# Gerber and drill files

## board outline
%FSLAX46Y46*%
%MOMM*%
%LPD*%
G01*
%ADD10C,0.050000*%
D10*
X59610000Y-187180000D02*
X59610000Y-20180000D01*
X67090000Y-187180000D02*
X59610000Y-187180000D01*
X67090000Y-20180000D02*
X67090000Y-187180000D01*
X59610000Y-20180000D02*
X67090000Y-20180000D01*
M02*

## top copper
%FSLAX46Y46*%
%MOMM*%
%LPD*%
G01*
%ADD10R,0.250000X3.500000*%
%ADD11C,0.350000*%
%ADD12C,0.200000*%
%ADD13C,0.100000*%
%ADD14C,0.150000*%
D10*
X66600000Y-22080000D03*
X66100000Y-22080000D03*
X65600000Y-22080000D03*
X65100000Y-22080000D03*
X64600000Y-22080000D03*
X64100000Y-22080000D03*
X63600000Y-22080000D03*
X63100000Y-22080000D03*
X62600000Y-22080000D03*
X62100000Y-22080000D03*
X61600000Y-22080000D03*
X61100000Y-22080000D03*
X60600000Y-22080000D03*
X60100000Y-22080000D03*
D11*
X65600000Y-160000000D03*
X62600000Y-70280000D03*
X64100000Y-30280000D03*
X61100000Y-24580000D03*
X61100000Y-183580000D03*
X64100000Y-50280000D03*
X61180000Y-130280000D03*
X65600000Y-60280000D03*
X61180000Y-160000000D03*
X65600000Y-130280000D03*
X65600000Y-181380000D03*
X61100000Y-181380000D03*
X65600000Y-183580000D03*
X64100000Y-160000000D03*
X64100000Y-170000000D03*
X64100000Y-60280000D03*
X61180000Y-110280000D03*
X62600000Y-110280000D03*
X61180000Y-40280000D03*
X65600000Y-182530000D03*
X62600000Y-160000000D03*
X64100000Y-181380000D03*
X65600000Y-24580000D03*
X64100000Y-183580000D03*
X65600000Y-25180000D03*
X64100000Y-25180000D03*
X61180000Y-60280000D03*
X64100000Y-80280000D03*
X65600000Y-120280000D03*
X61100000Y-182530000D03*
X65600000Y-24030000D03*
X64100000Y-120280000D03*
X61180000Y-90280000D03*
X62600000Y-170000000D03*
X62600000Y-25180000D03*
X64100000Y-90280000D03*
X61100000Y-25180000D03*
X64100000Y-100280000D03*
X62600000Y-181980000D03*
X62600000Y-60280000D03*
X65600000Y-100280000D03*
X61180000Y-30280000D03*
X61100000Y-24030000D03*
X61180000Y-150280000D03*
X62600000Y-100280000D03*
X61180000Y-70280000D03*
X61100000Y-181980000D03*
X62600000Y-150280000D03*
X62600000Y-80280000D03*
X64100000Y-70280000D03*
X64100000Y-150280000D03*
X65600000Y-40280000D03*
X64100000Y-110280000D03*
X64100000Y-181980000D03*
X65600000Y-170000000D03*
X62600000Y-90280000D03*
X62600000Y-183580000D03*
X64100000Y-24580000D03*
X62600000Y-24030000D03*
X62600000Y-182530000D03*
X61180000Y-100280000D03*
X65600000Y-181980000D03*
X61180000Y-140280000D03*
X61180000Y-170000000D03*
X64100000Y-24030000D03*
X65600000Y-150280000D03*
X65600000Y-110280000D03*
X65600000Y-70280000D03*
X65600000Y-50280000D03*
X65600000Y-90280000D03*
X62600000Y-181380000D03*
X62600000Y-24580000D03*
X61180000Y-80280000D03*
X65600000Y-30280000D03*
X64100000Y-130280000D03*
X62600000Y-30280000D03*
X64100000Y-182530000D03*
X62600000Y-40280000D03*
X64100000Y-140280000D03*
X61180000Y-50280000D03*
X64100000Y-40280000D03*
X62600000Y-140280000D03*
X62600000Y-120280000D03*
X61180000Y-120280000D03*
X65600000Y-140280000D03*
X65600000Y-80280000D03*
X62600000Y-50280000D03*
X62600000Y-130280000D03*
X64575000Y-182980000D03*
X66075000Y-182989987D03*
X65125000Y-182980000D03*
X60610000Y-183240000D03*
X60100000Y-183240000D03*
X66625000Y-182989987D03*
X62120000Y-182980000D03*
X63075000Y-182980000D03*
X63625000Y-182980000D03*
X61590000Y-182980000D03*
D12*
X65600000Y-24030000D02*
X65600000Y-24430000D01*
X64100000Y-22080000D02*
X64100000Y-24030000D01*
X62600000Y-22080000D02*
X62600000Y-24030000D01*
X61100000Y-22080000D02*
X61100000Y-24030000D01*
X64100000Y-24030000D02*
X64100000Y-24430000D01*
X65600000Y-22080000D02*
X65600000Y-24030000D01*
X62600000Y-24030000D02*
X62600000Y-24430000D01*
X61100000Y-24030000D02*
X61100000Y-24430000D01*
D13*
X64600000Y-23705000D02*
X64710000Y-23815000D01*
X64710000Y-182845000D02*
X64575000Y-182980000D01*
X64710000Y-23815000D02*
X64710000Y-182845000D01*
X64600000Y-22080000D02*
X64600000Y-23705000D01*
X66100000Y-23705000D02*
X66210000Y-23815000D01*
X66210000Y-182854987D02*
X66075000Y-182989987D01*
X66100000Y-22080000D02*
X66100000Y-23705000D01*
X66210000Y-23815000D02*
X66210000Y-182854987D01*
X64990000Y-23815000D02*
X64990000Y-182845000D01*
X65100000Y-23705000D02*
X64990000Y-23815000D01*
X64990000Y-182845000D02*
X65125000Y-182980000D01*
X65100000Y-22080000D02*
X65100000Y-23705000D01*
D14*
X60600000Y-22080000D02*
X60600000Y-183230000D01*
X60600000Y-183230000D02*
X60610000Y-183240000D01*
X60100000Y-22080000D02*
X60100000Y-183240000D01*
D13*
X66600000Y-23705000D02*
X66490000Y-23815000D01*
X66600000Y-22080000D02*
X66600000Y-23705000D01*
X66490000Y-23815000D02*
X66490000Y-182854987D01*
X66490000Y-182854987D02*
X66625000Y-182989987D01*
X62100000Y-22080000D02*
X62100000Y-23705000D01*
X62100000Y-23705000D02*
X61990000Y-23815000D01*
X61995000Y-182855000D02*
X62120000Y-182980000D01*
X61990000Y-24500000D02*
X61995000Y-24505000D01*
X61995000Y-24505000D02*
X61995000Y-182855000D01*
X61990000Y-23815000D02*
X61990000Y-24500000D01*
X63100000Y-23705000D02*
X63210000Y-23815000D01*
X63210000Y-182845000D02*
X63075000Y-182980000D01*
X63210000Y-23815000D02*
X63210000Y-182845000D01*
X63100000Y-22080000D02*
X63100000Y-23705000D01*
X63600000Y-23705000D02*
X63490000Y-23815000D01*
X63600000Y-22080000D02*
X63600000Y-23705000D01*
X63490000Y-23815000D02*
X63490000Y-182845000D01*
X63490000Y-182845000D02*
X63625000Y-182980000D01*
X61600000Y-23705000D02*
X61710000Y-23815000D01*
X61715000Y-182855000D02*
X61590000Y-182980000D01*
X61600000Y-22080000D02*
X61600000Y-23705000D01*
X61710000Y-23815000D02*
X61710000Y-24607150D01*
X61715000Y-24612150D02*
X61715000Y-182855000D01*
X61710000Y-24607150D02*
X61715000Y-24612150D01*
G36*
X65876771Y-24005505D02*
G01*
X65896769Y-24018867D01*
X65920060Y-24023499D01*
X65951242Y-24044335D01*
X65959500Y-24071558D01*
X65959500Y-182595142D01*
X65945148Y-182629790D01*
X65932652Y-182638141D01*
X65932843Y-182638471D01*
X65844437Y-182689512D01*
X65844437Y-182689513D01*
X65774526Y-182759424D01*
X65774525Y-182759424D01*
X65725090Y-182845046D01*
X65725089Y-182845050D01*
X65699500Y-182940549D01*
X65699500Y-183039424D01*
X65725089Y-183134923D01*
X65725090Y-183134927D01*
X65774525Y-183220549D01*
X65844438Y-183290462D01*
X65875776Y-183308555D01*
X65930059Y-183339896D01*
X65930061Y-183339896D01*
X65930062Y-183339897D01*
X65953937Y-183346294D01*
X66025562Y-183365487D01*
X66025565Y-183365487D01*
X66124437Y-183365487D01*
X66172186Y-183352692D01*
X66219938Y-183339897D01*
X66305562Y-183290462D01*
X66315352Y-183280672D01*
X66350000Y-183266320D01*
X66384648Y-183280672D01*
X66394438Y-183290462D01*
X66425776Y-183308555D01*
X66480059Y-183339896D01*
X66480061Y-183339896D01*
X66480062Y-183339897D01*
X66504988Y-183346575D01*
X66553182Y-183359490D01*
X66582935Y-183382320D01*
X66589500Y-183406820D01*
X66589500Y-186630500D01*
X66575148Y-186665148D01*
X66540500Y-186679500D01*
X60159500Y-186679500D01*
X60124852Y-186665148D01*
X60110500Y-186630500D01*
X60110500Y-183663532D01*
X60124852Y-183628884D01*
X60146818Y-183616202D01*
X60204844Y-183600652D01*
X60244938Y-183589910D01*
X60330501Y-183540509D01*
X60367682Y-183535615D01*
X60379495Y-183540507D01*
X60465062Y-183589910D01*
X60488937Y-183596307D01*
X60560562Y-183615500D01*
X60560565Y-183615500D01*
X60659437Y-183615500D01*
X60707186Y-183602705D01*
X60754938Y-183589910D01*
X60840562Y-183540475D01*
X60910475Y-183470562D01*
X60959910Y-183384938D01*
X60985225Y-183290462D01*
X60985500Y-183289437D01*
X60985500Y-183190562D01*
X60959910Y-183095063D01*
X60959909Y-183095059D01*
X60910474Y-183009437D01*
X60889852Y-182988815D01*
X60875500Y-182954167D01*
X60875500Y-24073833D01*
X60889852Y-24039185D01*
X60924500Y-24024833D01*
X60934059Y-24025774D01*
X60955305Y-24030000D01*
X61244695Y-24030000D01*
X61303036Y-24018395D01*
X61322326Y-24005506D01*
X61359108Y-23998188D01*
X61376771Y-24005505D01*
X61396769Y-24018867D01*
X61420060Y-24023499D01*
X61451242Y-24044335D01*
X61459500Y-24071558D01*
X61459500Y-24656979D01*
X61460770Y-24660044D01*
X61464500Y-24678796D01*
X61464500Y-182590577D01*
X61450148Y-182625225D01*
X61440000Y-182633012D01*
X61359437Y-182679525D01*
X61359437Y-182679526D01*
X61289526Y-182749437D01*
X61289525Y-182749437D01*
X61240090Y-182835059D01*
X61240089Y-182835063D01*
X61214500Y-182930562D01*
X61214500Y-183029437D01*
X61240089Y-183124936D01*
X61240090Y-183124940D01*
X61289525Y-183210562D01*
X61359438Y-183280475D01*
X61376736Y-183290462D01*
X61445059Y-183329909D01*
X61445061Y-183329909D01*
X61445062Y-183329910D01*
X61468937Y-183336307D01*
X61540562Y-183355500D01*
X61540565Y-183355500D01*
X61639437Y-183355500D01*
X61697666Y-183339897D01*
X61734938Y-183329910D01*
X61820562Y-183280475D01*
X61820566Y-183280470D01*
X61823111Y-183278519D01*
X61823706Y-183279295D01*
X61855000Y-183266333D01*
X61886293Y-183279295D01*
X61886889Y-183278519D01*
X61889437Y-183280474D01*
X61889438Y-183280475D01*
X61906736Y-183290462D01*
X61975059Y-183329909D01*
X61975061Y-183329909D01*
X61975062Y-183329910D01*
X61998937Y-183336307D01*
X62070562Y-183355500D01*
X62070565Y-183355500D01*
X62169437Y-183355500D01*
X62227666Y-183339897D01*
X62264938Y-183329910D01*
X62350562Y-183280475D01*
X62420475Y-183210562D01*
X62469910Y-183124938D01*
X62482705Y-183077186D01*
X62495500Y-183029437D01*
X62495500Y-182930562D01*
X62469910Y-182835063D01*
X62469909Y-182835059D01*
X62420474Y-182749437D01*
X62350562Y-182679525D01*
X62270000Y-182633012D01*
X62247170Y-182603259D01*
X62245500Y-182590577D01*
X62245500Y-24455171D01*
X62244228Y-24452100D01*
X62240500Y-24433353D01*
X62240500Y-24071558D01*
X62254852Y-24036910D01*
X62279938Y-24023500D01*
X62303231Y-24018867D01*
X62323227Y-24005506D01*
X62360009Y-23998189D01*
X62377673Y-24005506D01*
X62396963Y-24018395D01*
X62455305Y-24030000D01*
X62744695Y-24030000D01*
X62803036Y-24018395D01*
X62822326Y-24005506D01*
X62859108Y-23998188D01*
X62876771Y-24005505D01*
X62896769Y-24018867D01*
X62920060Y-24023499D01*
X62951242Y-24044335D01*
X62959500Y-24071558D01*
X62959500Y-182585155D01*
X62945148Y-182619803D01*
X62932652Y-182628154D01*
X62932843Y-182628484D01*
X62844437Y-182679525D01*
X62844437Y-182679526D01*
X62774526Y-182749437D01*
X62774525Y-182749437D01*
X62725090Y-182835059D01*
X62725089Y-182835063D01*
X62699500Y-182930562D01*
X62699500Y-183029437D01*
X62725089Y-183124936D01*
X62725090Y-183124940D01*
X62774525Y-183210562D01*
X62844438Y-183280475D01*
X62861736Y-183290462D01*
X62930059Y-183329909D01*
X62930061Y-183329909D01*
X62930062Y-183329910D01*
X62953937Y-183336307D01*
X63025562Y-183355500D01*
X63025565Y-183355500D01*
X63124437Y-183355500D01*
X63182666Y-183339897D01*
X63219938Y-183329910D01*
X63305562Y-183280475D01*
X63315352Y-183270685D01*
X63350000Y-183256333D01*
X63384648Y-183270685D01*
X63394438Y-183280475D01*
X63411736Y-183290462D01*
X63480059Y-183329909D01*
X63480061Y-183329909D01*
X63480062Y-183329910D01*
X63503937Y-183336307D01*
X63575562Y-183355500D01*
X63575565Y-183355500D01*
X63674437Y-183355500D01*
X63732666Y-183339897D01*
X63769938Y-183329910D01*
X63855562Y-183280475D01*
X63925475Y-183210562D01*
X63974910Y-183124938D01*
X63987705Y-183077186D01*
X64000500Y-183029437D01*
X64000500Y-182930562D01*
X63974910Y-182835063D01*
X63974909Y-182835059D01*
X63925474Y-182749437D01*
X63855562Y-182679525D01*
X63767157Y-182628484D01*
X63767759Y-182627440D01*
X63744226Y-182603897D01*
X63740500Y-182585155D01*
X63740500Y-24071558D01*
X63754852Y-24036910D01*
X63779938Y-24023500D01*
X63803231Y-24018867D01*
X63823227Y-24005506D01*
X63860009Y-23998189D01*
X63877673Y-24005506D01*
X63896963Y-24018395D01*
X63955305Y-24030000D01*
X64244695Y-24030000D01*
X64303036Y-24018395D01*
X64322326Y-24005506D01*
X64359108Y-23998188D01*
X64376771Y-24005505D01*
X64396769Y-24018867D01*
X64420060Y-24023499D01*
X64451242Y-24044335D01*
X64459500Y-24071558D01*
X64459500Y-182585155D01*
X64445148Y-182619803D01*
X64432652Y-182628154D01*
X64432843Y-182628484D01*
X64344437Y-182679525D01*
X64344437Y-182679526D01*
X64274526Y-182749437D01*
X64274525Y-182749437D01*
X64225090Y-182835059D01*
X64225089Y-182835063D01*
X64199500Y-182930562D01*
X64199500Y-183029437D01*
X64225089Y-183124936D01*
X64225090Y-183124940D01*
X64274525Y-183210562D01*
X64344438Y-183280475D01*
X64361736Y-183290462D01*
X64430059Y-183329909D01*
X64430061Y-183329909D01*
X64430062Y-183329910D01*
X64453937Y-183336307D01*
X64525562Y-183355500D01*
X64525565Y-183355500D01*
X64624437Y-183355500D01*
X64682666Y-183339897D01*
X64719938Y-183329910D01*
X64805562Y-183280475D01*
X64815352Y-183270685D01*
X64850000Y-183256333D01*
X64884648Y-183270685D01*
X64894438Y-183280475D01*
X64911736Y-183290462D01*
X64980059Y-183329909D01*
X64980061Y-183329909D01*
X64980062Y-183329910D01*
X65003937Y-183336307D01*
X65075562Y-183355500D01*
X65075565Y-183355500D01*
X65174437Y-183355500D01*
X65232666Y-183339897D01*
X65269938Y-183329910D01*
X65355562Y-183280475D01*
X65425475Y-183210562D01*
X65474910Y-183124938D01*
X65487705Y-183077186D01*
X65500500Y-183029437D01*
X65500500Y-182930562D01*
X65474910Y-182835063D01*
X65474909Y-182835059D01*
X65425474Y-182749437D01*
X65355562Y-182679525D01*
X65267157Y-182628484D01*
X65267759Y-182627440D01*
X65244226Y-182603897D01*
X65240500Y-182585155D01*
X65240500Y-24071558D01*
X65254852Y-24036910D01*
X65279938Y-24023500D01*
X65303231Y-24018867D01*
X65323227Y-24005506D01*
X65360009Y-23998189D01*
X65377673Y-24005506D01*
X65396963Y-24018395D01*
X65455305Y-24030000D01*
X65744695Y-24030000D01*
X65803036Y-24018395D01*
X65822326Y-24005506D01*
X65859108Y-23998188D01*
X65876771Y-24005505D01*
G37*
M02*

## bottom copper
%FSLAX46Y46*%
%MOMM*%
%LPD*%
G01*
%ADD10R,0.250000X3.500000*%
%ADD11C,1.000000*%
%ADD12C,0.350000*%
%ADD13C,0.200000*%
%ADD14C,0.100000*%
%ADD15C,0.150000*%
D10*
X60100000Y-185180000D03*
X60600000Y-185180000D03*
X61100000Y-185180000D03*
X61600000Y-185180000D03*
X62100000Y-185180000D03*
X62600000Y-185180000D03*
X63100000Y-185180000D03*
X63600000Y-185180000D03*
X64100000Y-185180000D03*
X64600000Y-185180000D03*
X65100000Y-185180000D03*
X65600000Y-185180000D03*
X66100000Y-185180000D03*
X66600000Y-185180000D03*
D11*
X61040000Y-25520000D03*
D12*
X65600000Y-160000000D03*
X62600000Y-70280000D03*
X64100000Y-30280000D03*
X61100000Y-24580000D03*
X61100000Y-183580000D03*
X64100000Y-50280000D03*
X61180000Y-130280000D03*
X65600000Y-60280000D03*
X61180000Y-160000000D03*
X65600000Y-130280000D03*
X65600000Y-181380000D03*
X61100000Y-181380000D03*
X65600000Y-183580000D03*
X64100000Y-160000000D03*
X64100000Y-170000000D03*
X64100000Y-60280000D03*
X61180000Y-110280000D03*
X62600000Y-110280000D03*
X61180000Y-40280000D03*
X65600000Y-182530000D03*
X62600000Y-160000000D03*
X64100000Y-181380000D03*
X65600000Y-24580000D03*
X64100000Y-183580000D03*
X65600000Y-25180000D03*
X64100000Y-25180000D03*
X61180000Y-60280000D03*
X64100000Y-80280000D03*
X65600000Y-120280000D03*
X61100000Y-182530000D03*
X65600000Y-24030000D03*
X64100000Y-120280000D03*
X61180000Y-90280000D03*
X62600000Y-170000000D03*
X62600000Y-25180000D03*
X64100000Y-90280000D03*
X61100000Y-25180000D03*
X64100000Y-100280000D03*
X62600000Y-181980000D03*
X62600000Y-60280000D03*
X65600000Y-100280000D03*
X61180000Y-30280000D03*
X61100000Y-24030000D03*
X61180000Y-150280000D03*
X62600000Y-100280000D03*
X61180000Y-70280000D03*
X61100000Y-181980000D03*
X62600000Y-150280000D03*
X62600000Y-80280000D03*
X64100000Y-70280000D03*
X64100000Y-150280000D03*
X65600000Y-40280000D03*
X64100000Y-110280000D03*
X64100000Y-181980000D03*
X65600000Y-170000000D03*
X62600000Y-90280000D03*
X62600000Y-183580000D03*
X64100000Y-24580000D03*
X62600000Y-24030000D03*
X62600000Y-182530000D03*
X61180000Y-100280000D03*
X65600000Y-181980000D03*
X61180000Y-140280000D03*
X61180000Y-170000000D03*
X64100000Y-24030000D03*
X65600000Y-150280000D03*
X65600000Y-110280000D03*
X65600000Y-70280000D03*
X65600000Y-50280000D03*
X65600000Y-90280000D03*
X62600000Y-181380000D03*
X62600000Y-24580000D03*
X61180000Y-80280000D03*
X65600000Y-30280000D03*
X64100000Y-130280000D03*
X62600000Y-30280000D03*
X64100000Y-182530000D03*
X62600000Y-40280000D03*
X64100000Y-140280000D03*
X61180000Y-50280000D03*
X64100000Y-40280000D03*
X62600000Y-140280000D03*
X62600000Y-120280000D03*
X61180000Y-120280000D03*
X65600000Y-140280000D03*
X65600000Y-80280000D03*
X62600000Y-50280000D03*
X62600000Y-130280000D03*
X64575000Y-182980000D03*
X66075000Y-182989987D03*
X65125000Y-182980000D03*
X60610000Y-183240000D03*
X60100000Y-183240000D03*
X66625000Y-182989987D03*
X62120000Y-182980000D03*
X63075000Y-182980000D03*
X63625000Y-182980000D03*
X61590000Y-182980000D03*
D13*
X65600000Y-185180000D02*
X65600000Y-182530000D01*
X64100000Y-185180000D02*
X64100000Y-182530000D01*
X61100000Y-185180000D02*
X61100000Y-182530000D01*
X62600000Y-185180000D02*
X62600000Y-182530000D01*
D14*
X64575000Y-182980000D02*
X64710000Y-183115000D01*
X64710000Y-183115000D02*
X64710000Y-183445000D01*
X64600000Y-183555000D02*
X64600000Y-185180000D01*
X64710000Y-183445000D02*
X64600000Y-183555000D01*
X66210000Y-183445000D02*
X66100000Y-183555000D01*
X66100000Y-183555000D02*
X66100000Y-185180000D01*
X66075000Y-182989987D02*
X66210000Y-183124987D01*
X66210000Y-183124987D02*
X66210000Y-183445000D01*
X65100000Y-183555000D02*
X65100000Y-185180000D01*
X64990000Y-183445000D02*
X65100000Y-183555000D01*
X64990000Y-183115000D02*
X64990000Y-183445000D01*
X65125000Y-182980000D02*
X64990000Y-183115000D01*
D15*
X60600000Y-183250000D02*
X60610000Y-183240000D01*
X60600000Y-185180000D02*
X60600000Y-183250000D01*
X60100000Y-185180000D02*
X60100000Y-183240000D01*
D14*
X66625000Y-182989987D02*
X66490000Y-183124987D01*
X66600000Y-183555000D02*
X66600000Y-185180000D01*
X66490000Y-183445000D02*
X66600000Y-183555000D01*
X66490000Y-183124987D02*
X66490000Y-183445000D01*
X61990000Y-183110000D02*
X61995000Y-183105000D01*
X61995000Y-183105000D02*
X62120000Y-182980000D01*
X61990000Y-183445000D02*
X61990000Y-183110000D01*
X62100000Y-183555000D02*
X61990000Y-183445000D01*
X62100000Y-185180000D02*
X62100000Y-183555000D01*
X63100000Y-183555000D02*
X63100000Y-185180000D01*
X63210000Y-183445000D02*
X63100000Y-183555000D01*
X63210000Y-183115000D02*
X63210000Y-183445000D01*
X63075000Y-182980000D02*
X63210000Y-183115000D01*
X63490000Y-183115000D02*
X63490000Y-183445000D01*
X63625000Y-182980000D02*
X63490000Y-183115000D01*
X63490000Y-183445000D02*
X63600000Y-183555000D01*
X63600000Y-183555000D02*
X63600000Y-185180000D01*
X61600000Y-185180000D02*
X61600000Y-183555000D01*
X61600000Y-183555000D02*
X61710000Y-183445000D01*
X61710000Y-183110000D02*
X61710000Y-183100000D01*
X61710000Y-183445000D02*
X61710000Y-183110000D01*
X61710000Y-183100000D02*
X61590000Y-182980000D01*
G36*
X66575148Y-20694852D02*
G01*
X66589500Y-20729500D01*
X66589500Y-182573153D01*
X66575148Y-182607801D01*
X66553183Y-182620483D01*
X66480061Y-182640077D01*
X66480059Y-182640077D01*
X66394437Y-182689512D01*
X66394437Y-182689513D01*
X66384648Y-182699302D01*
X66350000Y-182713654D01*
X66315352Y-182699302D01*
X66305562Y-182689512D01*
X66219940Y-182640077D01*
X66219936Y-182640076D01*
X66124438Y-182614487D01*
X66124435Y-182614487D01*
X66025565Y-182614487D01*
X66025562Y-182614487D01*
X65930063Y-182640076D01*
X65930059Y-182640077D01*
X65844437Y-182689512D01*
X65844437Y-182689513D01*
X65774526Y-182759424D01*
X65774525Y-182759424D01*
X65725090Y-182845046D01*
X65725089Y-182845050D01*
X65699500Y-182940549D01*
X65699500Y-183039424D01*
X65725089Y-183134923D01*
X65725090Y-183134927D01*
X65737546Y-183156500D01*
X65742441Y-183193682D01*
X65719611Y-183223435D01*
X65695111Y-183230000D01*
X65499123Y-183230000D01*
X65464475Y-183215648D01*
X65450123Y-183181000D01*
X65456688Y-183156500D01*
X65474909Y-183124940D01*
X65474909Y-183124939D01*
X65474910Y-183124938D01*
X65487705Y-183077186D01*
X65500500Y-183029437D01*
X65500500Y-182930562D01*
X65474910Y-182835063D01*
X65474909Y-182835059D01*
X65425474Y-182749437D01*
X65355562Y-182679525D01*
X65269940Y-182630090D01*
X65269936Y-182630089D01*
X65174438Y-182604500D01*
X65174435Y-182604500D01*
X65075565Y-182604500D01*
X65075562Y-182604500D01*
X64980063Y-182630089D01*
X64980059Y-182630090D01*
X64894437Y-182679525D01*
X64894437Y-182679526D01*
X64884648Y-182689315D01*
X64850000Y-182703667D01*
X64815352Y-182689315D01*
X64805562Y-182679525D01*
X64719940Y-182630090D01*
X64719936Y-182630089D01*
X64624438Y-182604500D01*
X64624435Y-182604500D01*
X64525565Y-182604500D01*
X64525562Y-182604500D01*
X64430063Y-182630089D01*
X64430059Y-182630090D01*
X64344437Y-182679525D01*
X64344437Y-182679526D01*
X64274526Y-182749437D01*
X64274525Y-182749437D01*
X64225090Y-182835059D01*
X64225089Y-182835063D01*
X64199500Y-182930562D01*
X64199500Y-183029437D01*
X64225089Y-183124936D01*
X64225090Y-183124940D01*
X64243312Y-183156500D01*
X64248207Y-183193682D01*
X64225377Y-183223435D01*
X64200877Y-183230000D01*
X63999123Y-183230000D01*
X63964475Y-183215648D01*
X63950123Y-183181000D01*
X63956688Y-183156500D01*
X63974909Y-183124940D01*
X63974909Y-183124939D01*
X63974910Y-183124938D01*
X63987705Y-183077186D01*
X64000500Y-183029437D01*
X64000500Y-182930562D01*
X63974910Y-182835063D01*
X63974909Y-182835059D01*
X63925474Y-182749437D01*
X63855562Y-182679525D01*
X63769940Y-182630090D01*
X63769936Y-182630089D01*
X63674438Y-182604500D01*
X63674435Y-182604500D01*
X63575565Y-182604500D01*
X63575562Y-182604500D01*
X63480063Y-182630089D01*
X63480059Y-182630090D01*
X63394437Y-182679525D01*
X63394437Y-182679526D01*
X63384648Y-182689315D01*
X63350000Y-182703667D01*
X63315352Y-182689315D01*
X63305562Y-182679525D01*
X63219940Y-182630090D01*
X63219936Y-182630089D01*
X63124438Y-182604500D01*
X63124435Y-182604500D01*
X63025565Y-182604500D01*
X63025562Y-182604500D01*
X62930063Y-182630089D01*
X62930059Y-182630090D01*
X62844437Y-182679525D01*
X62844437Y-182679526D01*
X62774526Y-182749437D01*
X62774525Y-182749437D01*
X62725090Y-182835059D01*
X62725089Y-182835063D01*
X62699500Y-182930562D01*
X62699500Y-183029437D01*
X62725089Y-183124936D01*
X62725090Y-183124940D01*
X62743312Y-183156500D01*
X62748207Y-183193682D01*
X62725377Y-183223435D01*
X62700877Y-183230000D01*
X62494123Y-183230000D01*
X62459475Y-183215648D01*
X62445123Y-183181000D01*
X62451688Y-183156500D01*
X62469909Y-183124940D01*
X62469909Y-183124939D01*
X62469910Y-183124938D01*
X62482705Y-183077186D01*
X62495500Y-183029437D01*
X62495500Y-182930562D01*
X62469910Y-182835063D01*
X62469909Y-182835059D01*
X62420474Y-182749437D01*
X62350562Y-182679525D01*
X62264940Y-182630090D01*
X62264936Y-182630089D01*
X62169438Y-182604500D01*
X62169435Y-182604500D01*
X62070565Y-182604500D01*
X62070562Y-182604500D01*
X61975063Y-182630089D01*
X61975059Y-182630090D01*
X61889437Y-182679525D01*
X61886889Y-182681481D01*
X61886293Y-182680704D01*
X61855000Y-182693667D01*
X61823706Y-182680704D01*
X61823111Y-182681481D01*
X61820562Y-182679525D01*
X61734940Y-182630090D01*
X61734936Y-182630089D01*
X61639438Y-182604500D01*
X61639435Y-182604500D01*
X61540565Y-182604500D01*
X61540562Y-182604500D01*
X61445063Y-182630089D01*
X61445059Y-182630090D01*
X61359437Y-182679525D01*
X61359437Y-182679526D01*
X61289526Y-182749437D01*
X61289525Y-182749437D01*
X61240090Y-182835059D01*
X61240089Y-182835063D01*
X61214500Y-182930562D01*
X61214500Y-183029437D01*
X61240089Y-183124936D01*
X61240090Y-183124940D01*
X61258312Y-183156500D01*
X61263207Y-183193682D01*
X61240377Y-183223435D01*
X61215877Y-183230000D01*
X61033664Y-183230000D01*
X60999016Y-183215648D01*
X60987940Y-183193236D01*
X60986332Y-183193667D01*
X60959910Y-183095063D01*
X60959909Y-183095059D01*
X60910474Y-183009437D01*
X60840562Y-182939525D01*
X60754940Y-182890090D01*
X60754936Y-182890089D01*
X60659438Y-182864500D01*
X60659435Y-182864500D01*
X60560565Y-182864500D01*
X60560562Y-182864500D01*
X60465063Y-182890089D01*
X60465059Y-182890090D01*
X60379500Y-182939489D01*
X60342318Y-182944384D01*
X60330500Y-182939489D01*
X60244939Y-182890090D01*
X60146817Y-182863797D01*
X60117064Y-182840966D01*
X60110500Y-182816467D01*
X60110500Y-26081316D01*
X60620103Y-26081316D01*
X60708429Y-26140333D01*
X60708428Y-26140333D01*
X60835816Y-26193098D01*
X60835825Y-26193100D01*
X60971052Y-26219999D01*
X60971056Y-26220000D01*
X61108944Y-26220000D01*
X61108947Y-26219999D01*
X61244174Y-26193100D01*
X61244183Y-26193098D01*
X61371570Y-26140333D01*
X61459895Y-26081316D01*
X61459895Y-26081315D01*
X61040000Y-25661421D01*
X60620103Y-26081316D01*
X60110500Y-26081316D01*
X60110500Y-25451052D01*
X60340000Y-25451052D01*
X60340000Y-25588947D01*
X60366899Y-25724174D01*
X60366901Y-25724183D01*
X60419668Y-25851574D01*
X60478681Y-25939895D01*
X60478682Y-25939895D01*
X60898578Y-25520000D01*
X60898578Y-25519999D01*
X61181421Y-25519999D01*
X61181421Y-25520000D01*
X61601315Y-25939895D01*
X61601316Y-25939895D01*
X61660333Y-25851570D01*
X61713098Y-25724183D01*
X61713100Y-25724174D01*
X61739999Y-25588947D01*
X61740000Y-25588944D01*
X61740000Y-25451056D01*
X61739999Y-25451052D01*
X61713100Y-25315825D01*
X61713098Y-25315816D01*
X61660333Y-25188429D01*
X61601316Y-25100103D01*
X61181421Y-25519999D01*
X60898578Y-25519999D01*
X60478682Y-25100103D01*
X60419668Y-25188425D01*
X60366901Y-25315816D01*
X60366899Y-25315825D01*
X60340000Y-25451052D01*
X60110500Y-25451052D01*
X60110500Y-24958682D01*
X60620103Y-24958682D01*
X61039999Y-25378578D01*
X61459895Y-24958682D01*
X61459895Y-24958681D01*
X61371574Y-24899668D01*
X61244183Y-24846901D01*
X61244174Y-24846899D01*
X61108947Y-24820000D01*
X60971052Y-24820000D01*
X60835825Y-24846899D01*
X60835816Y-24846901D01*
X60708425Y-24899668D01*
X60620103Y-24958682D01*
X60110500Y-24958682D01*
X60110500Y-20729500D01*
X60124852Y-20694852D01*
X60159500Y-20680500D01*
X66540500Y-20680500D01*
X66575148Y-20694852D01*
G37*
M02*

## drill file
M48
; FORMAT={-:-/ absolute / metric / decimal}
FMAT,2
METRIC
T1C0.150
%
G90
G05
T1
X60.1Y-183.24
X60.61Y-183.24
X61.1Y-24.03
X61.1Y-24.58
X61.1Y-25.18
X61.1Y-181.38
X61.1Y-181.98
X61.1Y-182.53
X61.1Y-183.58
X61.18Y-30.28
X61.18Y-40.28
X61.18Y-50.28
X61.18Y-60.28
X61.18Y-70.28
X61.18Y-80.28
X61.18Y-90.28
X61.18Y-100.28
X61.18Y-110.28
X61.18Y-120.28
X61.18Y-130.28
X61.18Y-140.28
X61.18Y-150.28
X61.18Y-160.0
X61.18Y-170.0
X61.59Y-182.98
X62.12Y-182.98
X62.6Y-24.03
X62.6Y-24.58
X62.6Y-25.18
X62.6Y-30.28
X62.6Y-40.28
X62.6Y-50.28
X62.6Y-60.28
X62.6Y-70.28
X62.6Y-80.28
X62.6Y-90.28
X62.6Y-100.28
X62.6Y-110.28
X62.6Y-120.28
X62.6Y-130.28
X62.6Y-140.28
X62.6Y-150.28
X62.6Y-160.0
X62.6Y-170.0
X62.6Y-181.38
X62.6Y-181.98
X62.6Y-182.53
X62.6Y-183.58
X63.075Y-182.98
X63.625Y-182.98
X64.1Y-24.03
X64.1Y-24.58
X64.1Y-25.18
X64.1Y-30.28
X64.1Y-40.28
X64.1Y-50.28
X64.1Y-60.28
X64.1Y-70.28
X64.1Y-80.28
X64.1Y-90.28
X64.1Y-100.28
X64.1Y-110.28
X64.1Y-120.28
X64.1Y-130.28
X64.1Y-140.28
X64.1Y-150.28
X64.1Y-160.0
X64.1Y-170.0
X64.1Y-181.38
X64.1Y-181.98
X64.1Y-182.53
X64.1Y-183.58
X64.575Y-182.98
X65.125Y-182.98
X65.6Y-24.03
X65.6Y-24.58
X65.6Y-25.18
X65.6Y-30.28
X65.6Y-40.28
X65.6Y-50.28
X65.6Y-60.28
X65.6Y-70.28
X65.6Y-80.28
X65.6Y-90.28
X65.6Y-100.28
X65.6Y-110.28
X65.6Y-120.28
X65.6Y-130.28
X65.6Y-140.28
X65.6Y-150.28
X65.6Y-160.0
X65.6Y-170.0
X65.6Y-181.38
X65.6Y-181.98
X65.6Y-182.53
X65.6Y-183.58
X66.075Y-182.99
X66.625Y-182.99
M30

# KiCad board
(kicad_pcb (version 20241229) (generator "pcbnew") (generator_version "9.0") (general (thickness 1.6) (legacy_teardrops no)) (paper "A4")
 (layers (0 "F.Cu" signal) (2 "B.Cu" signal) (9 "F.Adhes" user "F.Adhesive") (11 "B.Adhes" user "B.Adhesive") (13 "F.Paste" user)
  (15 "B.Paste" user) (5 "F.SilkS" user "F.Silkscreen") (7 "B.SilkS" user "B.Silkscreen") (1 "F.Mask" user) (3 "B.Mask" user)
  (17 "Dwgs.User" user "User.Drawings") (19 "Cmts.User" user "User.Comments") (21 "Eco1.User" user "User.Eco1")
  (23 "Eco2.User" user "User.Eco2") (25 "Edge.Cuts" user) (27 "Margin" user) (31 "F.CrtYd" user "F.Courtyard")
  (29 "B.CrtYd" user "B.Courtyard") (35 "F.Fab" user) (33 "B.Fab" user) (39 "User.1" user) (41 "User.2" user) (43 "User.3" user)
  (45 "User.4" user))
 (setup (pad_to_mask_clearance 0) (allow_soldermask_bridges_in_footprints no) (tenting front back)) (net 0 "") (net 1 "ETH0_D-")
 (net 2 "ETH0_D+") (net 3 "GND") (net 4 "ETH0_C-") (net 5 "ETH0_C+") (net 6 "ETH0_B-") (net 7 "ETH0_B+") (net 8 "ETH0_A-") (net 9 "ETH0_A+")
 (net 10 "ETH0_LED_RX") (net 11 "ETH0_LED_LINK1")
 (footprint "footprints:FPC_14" (layer "F.Cu") (at 63.35 22.08)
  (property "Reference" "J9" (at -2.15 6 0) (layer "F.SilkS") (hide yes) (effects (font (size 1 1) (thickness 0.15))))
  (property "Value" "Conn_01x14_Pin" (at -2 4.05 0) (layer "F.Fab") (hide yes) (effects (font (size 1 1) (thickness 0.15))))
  (pad "1" smd rect (at 3.25 0) (size 0.25 3.5) (layers "F.Cu" "F.Mask" "F.Paste") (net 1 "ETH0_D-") (thermal_bridge_angle 45))
  (pad "2" smd rect (at 2.75 0) (size 0.25 3.5) (layers "F.Cu" "F.Mask" "F.Paste") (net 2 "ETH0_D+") (thermal_bridge_angle 45))
  (pad "3" smd rect (at 2.25 0) (size 0.25 3.5) (layers "F.Cu" "F.Mask" "F.Paste") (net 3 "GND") (thermal_bridge_angle 45))
  (pad "4" smd rect (at 1.75 0) (size 0.25 3.5) (layers "F.Cu" "F.Mask" "F.Paste") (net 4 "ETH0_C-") (thermal_bridge_angle 45))
  (pad "5" smd rect (at 1.25 0) (size 0.25 3.5) (layers "F.Cu" "F.Mask" "F.Paste") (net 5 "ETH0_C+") (thermal_bridge_angle 45))
  (pad "6" smd rect (at 0.75 0) (size 0.25 3.5) (layers "F.Cu" "F.Mask" "F.Paste") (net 3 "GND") (thermal_bridge_angle 45))
  (pad "7" smd rect (at 0.25 0) (size 0.25 3.5) (layers "F.Cu" "F.Mask" "F.Paste") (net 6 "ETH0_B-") (thermal_bridge_angle 45))
  (pad "8" smd rect (at -0.25 0) (size 0.25 3.5) (layers "F.Cu" "F.Mask" "F.Paste") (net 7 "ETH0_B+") (thermal_bridge_angle 45))
  (pad "9" smd rect (at -0.75 0) (size 0.25 3.5) (layers "F.Cu" "F.Mask" "F.Paste") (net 3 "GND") (thermal_bridge_angle 45))
  (pad "10" smd rect (at -1.25 0) (size 0.25 3.5) (layers "F.Cu" "F.Mask" "F.Paste") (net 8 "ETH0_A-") (thermal_bridge_angle 45))
  (pad "11" smd rect (at -1.75 0) (size 0.25 3.5) (layers "F.Cu" "F.Mask" "F.Paste") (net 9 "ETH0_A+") (thermal_bridge_angle 45))
  (pad "12" smd rect (at -2.25 0) (size 0.25 3.5) (layers "F.Cu" "F.Mask" "F.Paste") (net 3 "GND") (thermal_bridge_angle 45))
  (pad "13" smd rect (at -2.75 0) (size 0.25 3.5) (layers "F.Cu" "F.Mask" "F.Paste") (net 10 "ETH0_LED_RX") (thermal_bridge_angle 45))
  (pad "14" smd rect (at -3.25 0) (size 0.25 3.5) (layers "F.Cu" "F.Mask" "F.Paste") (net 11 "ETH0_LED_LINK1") (thermal_bridge_angle 45)))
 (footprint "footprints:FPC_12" (layer "B.Cu") (at 63.35 185.18 180)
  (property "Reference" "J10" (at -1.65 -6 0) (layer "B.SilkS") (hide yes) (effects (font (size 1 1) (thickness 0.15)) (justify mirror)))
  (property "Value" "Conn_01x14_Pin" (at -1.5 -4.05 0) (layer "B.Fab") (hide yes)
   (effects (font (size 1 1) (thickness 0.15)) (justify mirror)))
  (pad "1" smd rect (at 3.25 0 180) (size 0.25 3.5) (layers "B.Cu" "B.Mask" "B.Paste") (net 11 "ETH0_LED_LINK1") (thermal_bridge_angle 45))
  (pad "2" smd rect (at 2.75 0 180) (size 0.25 3.5) (layers "B.Cu" "B.Mask" "B.Paste") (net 10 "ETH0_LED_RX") (thermal_bridge_angle 45))
  (pad "3" smd rect (at 2.25 0 180) (size 0.25 3.5) (layers "B.Cu" "B.Mask" "B.Paste") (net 3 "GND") (thermal_bridge_angle 45))
  (pad "4" smd rect (at 1.75 0 180) (size 0.25 3.5) (layers "B.Cu" "B.Mask" "B.Paste") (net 9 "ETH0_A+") (thermal_bridge_angle 45))
  (pad "5" smd rect (at 1.25 0 180) (size 0.25 3.5) (layers "B.Cu" "B.Mask" "B.Paste") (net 8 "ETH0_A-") (thermal_bridge_angle 45))
  (pad "6" smd rect (at 0.75 0 180) (size 0.25 3.5) (layers "B.Cu" "B.Mask" "B.Paste") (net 3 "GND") (thermal_bridge_angle 45))
  (pad "7" smd rect (at 0.25 0 180) (size 0.25 3.5) (layers "B.Cu" "B.Mask" "B.Paste") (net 7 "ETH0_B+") (thermal_bridge_angle 45))
  (pad "8" smd rect (at -0.25 0 180) (size 0.25 3.5) (layers "B.Cu" "B.Mask" "B.Paste") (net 6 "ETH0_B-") (thermal_bridge_angle 45))
  (pad "9" smd rect (at -0.75 0 180) (size 0.25 3.5) (layers "B.Cu" "B.Mask" "B.Paste") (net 3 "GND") (thermal_bridge_angle 45))
  (pad "10" smd rect (at -1.25 0 180) (size 0.25 3.5) (layers "B.Cu" "B.Mask" "B.Paste") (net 5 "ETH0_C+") (thermal_bridge_angle 45))
  (pad "11" smd rect (at -1.75 0 180) (size 0.25 3.5) (layers "B.Cu" "B.Mask" "B.Paste") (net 4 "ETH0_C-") (thermal_bridge_angle 45))
  (pad "12" smd rect (at -2.25 0 180) (size 0.25 3.5) (layers "B.Cu" "B.Mask" "B.Paste") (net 3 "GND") (thermal_bridge_angle 45))
  (pad "13" smd rect (at -2.75 0 180) (size 0.25 3.5) (layers "B.Cu" "B.Mask" "B.Paste") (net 2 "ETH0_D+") (thermal_bridge_angle 45))
  (pad "14" smd rect (at -3.25 0 180) (size 0.25 3.5) (layers "B.Cu" "B.Mask" "B.Paste") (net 1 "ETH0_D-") (thermal_bridge_angle 45)))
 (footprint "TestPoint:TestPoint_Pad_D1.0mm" (layer "B.Cu") (at 61.04 25.52 180)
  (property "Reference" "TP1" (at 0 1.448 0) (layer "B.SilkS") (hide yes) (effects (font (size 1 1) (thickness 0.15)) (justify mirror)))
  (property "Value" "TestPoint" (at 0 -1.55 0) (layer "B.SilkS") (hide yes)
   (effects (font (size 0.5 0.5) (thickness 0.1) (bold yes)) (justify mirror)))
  (pad "1" smd circle (at 0 0 180) (size 1 1) (layers "B.Cu" "B.Mask") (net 3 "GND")))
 (gr_line (start 59.61 187.18) (end 59.61 20.18) (stroke (width 0.05) (type solid)) (layer "Edge.Cuts"))
 (gr_line (start 67.09 187.18) (end 59.61 187.18) (stroke (width 0.05) (type solid)) (layer "Edge.Cuts"))
 (gr_line (start 67.09 20.18) (end 67.09 187.18) (stroke (width 0.05) (type solid)) (layer "Edge.Cuts"))
 (gr_line (start 59.61 20.18) (end 67.09 20.18) (stroke (width 0.05) (type solid)) (layer "Edge.Cuts"))
 (segment (start 65.6 24.03) (end 65.6 24.43) (width 0.2) (layer "F.Cu") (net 3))
 (segment (start 64.1 22.08) (end 64.1 24.03) (width 0.2) (layer "F.Cu") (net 3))
 (segment (start 62.6 22.08) (end 62.6 24.03) (width 0.2) (layer "F.Cu") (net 3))
 (segment (start 61.1 22.08) (end 61.1 24.03) (width 0.2) (layer "F.Cu") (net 3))
 (segment (start 64.1 24.03) (end 64.1 24.43) (width 0.2) (layer "F.Cu") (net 3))
 (segment (start 65.6 22.08) (end 65.6 24.03) (width 0.2) (layer "F.Cu") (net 3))
 (segment (start 62.6 24.03) (end 62.6 24.43) (width 0.2) (layer "F.Cu") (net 3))
 (segment (start 61.1 24.03) (end 61.1 24.43) (width 0.2) (layer "F.Cu") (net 3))
 (via (at 65.6 160) (size 0.35) (drill 0.15) (layers "F.Cu" "B.Cu") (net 3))
 (via (at 62.6 70.28) (size 0.35) (drill 0.15) (layers "F.Cu" "B.Cu") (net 3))
 (via (at 64.1 30.28) (size 0.35) (drill 0.15) (layers "F.Cu" "B.Cu") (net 3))
 (via (at 61.1 24.58) (size 0.35) (drill 0.15) (layers "F.Cu" "B.Cu") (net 3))
 (via (at 61.1 183.58) (size 0.35) (drill 0.15) (layers "F.Cu" "B.Cu") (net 3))
 (via (at 64.1 50.28) (size 0.35) (drill 0.15) (layers "F.Cu" "B.Cu") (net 3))
 (via (at 61.18 130.28) (size 0.35) (drill 0.15) (layers "F.Cu" "B.Cu") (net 3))
 (via (at 65.6 60.28) (size 0.35) (drill 0.15) (layers "F.Cu" "B.Cu") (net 3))
 (via (at 61.18 160) (size 0.35) (drill 0.15) (layers "F.Cu" "B.Cu") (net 3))
 (via (at 65.6 130.28) (size 0.35) (drill 0.15) (layers "F.Cu" "B.Cu") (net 3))
 (via (at 65.6 181.38) (size 0.35) (drill 0.15) (layers "F.Cu" "B.Cu") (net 3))
 (via (at 61.1 181.38) (size 0.35) (drill 0.15) (layers "F.Cu" "B.Cu") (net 3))
 (via (at 65.6 183.58) (size 0.35) (drill 0.15) (layers "F.Cu" "B.Cu") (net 3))
 (via (at 64.1 160) (size 0.35) (drill 0.15) (layers "F.Cu" "B.Cu") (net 3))
 (via (at 64.1 170) (size 0.35) (drill 0.15) (layers "F.Cu" "B.Cu") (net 3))
 (via (at 64.1 60.28) (size 0.35) (drill 0.15) (layers "F.Cu" "B.Cu") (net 3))
 (via (at 61.18 110.28) (size 0.35) (drill 0.15) (layers "F.Cu" "B.Cu") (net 3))
 (via (at 62.6 110.28) (size 0.35) (drill 0.15) (layers "F.Cu" "B.Cu") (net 3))
 (via (at 61.18 40.28) (size 0.35) (drill 0.15) (layers "F.Cu" "B.Cu") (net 3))
 (via (at 65.6 182.53) (size 0.35) (drill 0.15) (layers "F.Cu" "B.Cu") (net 3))
 (via (at 62.6 160) (size 0.35) (drill 0.15) (layers "F.Cu" "B.Cu") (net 3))
 (via (at 64.1 181.38) (size 0.35) (drill 0.15) (layers "F.Cu" "B.Cu") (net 3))
 (via (at 65.6 24.58) (size 0.35) (drill 0.15) (layers "F.Cu" "B.Cu") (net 3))
 (via (at 64.1 183.58) (size 0.35) (drill 0.15) (layers "F.Cu" "B.Cu") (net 3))
 (via (at 65.6 25.18) (size 0.35) (drill 0.15) (layers "F.Cu" "B.Cu") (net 3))
 (via (at 64.1 25.18) (size 0.35) (drill 0.15) (layers "F.Cu" "B.Cu") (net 3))
 (via (at 61.18 60.28) (size 0.35) (drill 0.15) (layers "F.Cu" "B.Cu") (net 3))
 (via (at 64.1 80.28) (size 0.35) (drill 0.15) (layers "F.Cu" "B.Cu") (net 3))
 (via (at 65.6 120.28) (size 0.35) (drill 0.15) (layers "F.Cu" "B.Cu") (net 3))
 (via (at 61.1 182.53) (size 0.35) (drill 0.15) (layers "F.Cu" "B.Cu") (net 3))
 (via (at 65.6 24.03) (size 0.35) (drill 0.15) (layers "F.Cu" "B.Cu") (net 3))
 (via (at 64.1 120.28) (size 0.35) (drill 0.15) (layers "F.Cu" "B.Cu") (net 3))
 (via (at 61.18 90.28) (size 0.35) (drill 0.15) (layers "F.Cu" "B.Cu") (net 3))
 (via (at 62.6 170) (size 0.35) (drill 0.15) (layers "F.Cu" "B.Cu") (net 3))
 (via (at 62.6 25.18) (size 0.35) (drill 0.15) (layers "F.Cu" "B.Cu") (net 3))
 (via (at 64.1 90.28) (size 0.35) (drill 0.15) (layers "F.Cu" "B.Cu") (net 3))
 (via (at 61.1 25.18) (size 0.35) (drill 0.15) (layers "F.Cu" "B.Cu") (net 3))
 (via (at 64.1 100.28) (size 0.35) (drill 0.15) (layers "F.Cu" "B.Cu") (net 3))
 (via (at 62.6 181.98) (size 0.35) (drill 0.15) (layers "F.Cu" "B.Cu") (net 3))
 (via (at 62.6 60.28) (size 0.35) (drill 0.15) (layers "F.Cu" "B.Cu") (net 3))
 (via (at 65.6 100.28) (size 0.35) (drill 0.15) (layers "F.Cu" "B.Cu") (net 3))
 (via (at 61.18 30.28) (size 0.35) (drill 0.15) (layers "F.Cu" "B.Cu") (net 3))
 (via (at 61.1 24.03) (size 0.35) (drill 0.15) (layers "F.Cu" "B.Cu") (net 3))
 (via (at 61.18 150.28) (size 0.35) (drill 0.15) (layers "F.Cu" "B.Cu") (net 3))
 (via (at 62.6 100.28) (size 0.35) (drill 0.15) (layers "F.Cu" "B.Cu") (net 3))
 (via (at 61.18 70.28) (size 0.35) (drill 0.15) (layers "F.Cu" "B.Cu") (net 3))
 (via (at 61.1 181.98) (size 0.35) (drill 0.15) (layers "F.Cu" "B.Cu") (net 3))
 (via (at 62.6 150.28) (size 0.35) (drill 0.15) (layers "F.Cu" "B.Cu") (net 3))
 (via (at 62.6 80.28) (size 0.35) (drill 0.15) (layers "F.Cu" "B.Cu") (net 3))
 (via (at 64.1 70.28) (size 0.35) (drill 0.15) (layers "F.Cu" "B.Cu") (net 3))
 (via (at 64.1 150.28) (size 0.35) (drill 0.15) (layers "F.Cu" "B.Cu") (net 3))
 (via (at 65.6 40.28) (size 0.35) (drill 0.15) (layers "F.Cu" "B.Cu") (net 3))
 (via (at 64.1 110.28) (size 0.35) (drill 0.15) (layers "F.Cu" "B.Cu") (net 3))
 (via (at 64.1 181.98) (size 0.35) (drill 0.15) (layers "F.Cu" "B.Cu") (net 3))
 (via (at 65.6 170) (size 0.35) (drill 0.15) (layers "F.Cu" "B.Cu") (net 3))
 (via (at 62.6 90.28) (size 0.35) (drill 0.15) (layers "F.Cu" "B.Cu") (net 3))
 (via (at 62.6 183.58) (size 0.35) (drill 0.15) (layers "F.Cu" "B.Cu") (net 3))
 (via (at 64.1 24.58) (size 0.35) (drill 0.15) (layers "F.Cu" "B.Cu") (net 3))
 (via (at 62.6 24.03) (size 0.35) (drill 0.15) (layers "F.Cu" "B.Cu") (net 3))
 (via (at 62.6 182.53) (size 0.35) (drill 0.15) (layers "F.Cu" "B.Cu") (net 3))
 (via (at 61.18 100.28) (size 0.35) (drill 0.15) (layers "F.Cu" "B.Cu") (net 3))
 (via (at 65.6 181.98) (size 0.35) (drill 0.15) (layers "F.Cu" "B.Cu") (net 3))
 (via (at 61.18 140.28) (size 0.35) (drill 0.15) (layers "F.Cu" "B.Cu") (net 3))
 (via (at 61.18 170) (size 0.35) (drill 0.15) (layers "F.Cu" "B.Cu") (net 3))
 (via (at 64.1 24.03) (size 0.35) (drill 0.15) (layers "F.Cu" "B.Cu") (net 3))
 (via (at 65.6 150.28) (size 0.35) (drill 0.15) (layers "F.Cu" "B.Cu") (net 3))
 (via (at 65.6 110.28) (size 0.35) (drill 0.15) (layers "F.Cu" "B.Cu") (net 3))
 (via (at 65.6 70.28) (size 0.35) (drill 0.15) (layers "F.Cu" "B.Cu") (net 3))
 (via (at 65.6 50.28) (size 0.35) (drill 0.15) (layers "F.Cu" "B.Cu") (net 3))
 (via (at 65.6 90.28) (size 0.35) (drill 0.15) (layers "F.Cu" "B.Cu") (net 3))
 (via (at 62.6 181.38) (size 0.35) (drill 0.15) (layers "F.Cu" "B.Cu") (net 3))
 (via (at 62.6 24.58) (size 0.35) (drill 0.15) (layers "F.Cu" "B.Cu") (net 3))
 (via (at 61.18 80.28) (size 0.35) (drill 0.15) (layers "F.Cu" "B.Cu") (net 3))
 (via (at 65.6 30.28) (size 0.35) (drill 0.15) (layers "F.Cu" "B.Cu") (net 3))
 (via (at 64.1 130.28) (size 0.35) (drill 0.15) (layers "F.Cu" "B.Cu") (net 3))
 (via (at 62.6 30.28) (size 0.35) (drill 0.15) (layers "F.Cu" "B.Cu") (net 3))
 (via (at 64.1 182.53) (size 0.35) (drill 0.15) (layers "F.Cu" "B.Cu") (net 3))
 (via (at 62.6 40.28) (size 0.35) (drill 0.15) (layers "F.Cu" "B.Cu") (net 3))
 (via (at 64.1 140.28) (size 0.35) (drill 0.15) (layers "F.Cu" "B.Cu") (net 3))
 (via (at 61.18 50.28) (size 0.35) (drill 0.15) (layers "F.Cu" "B.Cu") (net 3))
 (via (at 64.1 40.28) (size 0.35) (drill 0.15) (layers "F.Cu" "B.Cu") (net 3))
 (via (at 62.6 140.28) (size 0.35) (drill 0.15) (layers "F.Cu" "B.Cu") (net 3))
 (via (at 62.6 120.28) (size 0.35) (drill 0.15) (layers "F.Cu" "B.Cu") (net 3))
 (via (at 61.18 120.28) (size 0.35) (drill 0.15) (layers "F.Cu" "B.Cu") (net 3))
 (via (at 65.6 140.28) (size 0.35) (drill 0.15) (layers "F.Cu" "B.Cu") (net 3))
 (via (at 65.6 80.28) (size 0.35) (drill 0.15) (layers "F.Cu" "B.Cu") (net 3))
 (via (at 62.6 50.28) (size 0.35) (drill 0.15) (layers "F.Cu" "B.Cu") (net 3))
 (via (at 62.6 130.28) (size 0.35) (drill 0.15) (layers "F.Cu" "B.Cu") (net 3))
 (segment (start 65.6 185.18) (end 65.6 182.53) (width 0.2) (layer "B.Cu") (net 3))
 (segment (start 64.1 185.18) (end 64.1 182.53) (width 0.2) (layer "B.Cu") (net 3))
 (segment (start 61.1 185.18) (end 61.1 182.53) (width 0.2) (layer "B.Cu") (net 3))
 (segment (start 62.6 185.18) (end 62.6 182.53) (width 0.2) (layer "B.Cu") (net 3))
 (segment (start 64.6 23.705) (end 64.71 23.815) (width 0.1) (layer "F.Cu") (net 5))
 (segment (start 64.71 182.845) (end 64.575 182.98) (width 0.1) (layer "F.Cu") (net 5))
 (segment (start 64.71 23.815) (end 64.71 182.845) (width 0.1) (layer "F.Cu") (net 5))
 (segment (start 64.6 22.08) (end 64.6 23.705) (width 0.1) (layer "F.Cu") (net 5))
 (via (at 64.575 182.98) (size 0.35) (drill 0.15) (layers "F.Cu" "B.Cu") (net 5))
 (segment (start 64.575 182.98) (end 64.71 183.115) (width 0.1) (layer "B.Cu") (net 5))
 (segment (start 64.71 183.115) (end 64.71 183.445) (width 0.1) (layer "B.Cu") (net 5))
 (segment (start 64.6 183.555) (end 64.6 185.18) (width 0.1) (layer "B.Cu") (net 5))
 (segment (start 64.71 183.445) (end 64.6 183.555) (width 0.1) (layer "B.Cu") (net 5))
 (segment (start 66.1 23.705) (end 66.21 23.815) (width 0.1) (layer "F.Cu") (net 2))
 (segment (start 66.21 182.854987) (end 66.075 182.989987) (width 0.1) (layer "F.Cu") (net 2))
 (segment (start 66.1 22.08) (end 66.1 23.705) (width 0.1) (layer "F.Cu") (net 2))
 (segment (start 66.21 23.815) (end 66.21 182.854987) (width 0.1) (layer "F.Cu") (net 2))
 (via (at 66.075 182.989987) (size 0.35) (drill 0.15) (layers "F.Cu" "B.Cu") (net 2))
 (segment (start 66.21 183.445) (end 66.1 183.555) (width 0.1) (layer "B.Cu") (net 2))
 (segment (start 66.1 183.555) (end 66.1 185.18) (width 0.1) (layer "B.Cu") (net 2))
 (segment (start 66.075 182.989987) (end 66.21 183.124987) (width 0.1) (layer "B.Cu") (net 2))
 (segment (start 66.21 183.124987) (end 66.21 183.445) (width 0.1) (layer "B.Cu") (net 2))
 (segment (start 64.99 23.815) (end 64.99 182.845) (width 0.1) (layer "F.Cu") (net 4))
 (segment (start 65.1 23.705) (end 64.99 23.815) (width 0.1) (layer "F.Cu") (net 4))
 (segment (start 64.99 182.845) (end 65.125 182.98) (width 0.1) (layer "F.Cu") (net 4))
 (segment (start 65.1 22.08) (end 65.1 23.705) (width 0.1) (layer "F.Cu") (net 4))
 (via (at 65.125 182.98) (size 0.35) (drill 0.15) (layers "F.Cu" "B.Cu") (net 4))
 (segment (start 65.1 183.555) (end 65.1 185.18) (width 0.1) (layer "B.Cu") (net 4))
 (segment (start 64.99 183.445) (end 65.1 183.555) (width 0.1) (layer "B.Cu") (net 4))
 (segment (start 64.99 183.115) (end 64.99 183.445) (width 0.1) (layer "B.Cu") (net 4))
 (segment (start 65.125 182.98) (end 64.99 183.115) (width 0.1) (layer "B.Cu") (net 4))
 (segment (start 60.6 22.08) (end 60.6 183.23) (width 0.15) (layer "F.Cu") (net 10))
 (segment (start 60.6 183.23) (end 60.61 183.24) (width 0.15) (layer "F.Cu") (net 10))
 (via (at 60.61 183.24) (size 0.35) (drill 0.15) (layers "F.Cu" "B.Cu") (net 10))
 (segment (start 60.6 183.25) (end 60.61 183.24) (width 0.15) (layer "B.Cu") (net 10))
 (segment (start 60.6 185.18) (end 60.6 183.25) (width 0.15) (layer "B.Cu") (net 10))
 (segment (start 60.1 22.08) (end 60.1 183.24) (width 0.15) (layer "F.Cu") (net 11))
 (via (at 60.1 183.24) (size 0.35) (drill 0.15) (layers "F.Cu" "B.Cu") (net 11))
 (segment (start 60.1 185.18) (end 60.1 183.24) (width 0.15) (layer "B.Cu") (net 11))
 (segment (start 66.6 23.705) (end 66.49 23.815) (width 0.1) (layer "F.Cu") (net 1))
 (segment (start 66.6 22.08) (end 66.6 23.705) (width 0.1) (layer "F.Cu") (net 1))
 (segment (start 66.49 23.815) (end 66.49 182.854987) (width 0.1) (layer "F.Cu") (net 1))
 (segment (start 66.49 182.854987) (end 66.625 182.989987) (width 0.1) (layer "F.Cu") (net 1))
 (via (at 66.625 182.989987) (size 0.35) (drill 0.15) (layers "F.Cu" "B.Cu") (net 1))
 (segment (start 66.625 182.989987) (end 66.49 183.124987) (width 0.1) (layer "B.Cu") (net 1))
 (segment (start 66.6 183.555) (end 66.6 185.18) (width 0.1) (layer "B.Cu") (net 1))
 (segment (start 66.49 183.445) (end 66.6 183.555) (width 0.1) (layer "B.Cu") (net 1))
 (segment (start 66.49 183.124987) (end 66.49 183.445) (width 0.1) (layer "B.Cu") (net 1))
 (segment (start 62.1 22.08) (end 62.1 23.705) (width 0.1) (layer "F.Cu") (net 8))
 (segment (start 62.1 23.705) (end 61.99 23.815) (width 0.1) (layer "F.Cu") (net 8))
 (segment (start 61.995 182.855) (end 62.12 182.98) (width 0.1) (layer "F.Cu") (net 8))
 (segment (start 61.99 24.5) (end 61.995 24.505) (width 0.1) (layer "F.Cu") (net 8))
 (segment (start 61.995 24.505) (end 61.995 182.855) (width 0.1) (layer "F.Cu") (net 8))
 (segment (start 61.99 23.815) (end 61.99 24.5) (width 0.1) (layer "F.Cu") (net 8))
 (via (at 62.12 182.98) (size 0.35) (drill 0.15) (layers "F.Cu" "B.Cu") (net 8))
 (segment (start 61.99 183.11) (end 61.995 183.105) (width 0.1) (layer "B.Cu") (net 8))
 (segment (start 61.995 183.105) (end 62.12 182.98) (width 0.1) (layer "B.Cu") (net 8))
 (segment (start 61.99 183.445) (end 61.99 183.11) (width 0.1) (layer "B.Cu") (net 8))
 (segment (start 62.1 183.555) (end 61.99 183.445) (width 0.1) (layer "B.Cu") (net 8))
 (segment (start 62.1 185.18) (end 62.1 183.555) (width 0.1) (layer "B.Cu") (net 8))
 (segment (start 63.1 23.705) (end 63.21 23.815) (width 0.1) (layer "F.Cu") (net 7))
 (segment (start 63.21 182.845) (end 63.075 182.98) (width 0.1) (layer "F.Cu") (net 7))
 (segment (start 63.21 23.815) (end 63.21 182.845) (width 0.1) (layer "F.Cu") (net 7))
 (segment (start 63.1 22.08) (end 63.1 23.705) (width 0.1) (layer "F.Cu") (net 7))
 (via (at 63.075 182.98) (size 0.35) (drill 0.15) (layers "F.Cu" "B.Cu") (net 7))
 (segment (start 63.1 183.555) (end 63.1 185.18) (width 0.1) (layer "B.Cu") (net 7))
 (segment (start 63.21 183.445) (end 63.1 183.555) (width 0.1) (layer "B.Cu") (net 7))
 (segment (start 63.21 183.115) (end 63.21 183.445) (width 0.1) (layer "B.Cu") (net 7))
 (segment (start 63.075 182.98) (end 63.21 183.115) (width 0.1) (layer "B.Cu") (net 7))
 (segment (start 63.6 23.705) (end 63.49 23.815) (width 0.1) (layer "F.Cu") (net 6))
 (segment (start 63.6 22.08) (end 63.6 23.705) (width 0.1) (layer "F.Cu") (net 6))
 (segment (start 63.49 23.815) (end 63.49 182.845) (width 0.1) (layer "F.Cu") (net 6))
 (segment (start 63.49 182.845) (end 63.625 182.98) (width 0.1) (layer "F.Cu") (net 6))
 (via (at 63.625 182.98) (size 0.35) (drill 0.15) (layers "F.Cu" "B.Cu") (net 6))
 (segment (start 63.49 183.115) (end 63.49 183.445) (width 0.1) (layer "B.Cu") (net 6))
 (segment (start 63.625 182.98) (end 63.49 183.115) (width 0.1) (layer "B.Cu") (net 6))
 (segment (start 63.49 183.445) (end 63.6 183.555) (width 0.1) (layer "B.Cu") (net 6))
 (segment (start 63.6 183.555) (end 63.6 185.18) (width 0.1) (layer "B.Cu") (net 6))
 (segment (start 61.6 23.705) (end 61.71 23.815) (width 0.1) (layer "F.Cu") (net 9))
 (segment (start 61.715 182.855) (end 61.59 182.98) (width 0.1) (layer "F.Cu") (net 9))
 (segment (start 61.6 22.08) (end 61.6 23.705) (width 0.1) (layer "F.Cu") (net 9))
 (segment (start 61.71 23.815) (end 61.71 24.60715) (width 0.1) (layer "F.Cu") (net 9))
 (segment (start 61.715 24.61215) (end 61.715 182.855) (width 0.1) (layer "F.Cu") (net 9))
 (segment (start 61.71 24.60715) (end 61.715 24.61215) (width 0.1) (layer "F.Cu") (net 9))
 (via (at 61.59 182.98) (size 0.35) (drill 0.15) (layers "F.Cu" "B.Cu") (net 9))
 (segment (start 61.6 185.18) (end 61.6 183.555) (width 0.1) (layer "B.Cu") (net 9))
 (segment (start 61.6 183.555) (end 61.71 183.445) (width 0.1) (layer "B.Cu") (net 9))
 (segment (start 61.71 183.11) (end 61.71 183.1) (width 0.1) (layer "B.Cu") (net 9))
 (segment (start 61.71 183.445) (end 61.71 183.11) (width 0.1) (layer "B.Cu") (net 9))
 (segment (start 61.71 183.1) (end 61.59 182.98) (width 0.1) (layer "B.Cu") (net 9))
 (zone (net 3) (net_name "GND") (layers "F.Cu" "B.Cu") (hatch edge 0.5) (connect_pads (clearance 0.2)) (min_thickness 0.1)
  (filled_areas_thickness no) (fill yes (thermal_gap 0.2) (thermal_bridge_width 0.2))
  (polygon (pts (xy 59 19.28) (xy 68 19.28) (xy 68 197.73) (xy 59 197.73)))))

